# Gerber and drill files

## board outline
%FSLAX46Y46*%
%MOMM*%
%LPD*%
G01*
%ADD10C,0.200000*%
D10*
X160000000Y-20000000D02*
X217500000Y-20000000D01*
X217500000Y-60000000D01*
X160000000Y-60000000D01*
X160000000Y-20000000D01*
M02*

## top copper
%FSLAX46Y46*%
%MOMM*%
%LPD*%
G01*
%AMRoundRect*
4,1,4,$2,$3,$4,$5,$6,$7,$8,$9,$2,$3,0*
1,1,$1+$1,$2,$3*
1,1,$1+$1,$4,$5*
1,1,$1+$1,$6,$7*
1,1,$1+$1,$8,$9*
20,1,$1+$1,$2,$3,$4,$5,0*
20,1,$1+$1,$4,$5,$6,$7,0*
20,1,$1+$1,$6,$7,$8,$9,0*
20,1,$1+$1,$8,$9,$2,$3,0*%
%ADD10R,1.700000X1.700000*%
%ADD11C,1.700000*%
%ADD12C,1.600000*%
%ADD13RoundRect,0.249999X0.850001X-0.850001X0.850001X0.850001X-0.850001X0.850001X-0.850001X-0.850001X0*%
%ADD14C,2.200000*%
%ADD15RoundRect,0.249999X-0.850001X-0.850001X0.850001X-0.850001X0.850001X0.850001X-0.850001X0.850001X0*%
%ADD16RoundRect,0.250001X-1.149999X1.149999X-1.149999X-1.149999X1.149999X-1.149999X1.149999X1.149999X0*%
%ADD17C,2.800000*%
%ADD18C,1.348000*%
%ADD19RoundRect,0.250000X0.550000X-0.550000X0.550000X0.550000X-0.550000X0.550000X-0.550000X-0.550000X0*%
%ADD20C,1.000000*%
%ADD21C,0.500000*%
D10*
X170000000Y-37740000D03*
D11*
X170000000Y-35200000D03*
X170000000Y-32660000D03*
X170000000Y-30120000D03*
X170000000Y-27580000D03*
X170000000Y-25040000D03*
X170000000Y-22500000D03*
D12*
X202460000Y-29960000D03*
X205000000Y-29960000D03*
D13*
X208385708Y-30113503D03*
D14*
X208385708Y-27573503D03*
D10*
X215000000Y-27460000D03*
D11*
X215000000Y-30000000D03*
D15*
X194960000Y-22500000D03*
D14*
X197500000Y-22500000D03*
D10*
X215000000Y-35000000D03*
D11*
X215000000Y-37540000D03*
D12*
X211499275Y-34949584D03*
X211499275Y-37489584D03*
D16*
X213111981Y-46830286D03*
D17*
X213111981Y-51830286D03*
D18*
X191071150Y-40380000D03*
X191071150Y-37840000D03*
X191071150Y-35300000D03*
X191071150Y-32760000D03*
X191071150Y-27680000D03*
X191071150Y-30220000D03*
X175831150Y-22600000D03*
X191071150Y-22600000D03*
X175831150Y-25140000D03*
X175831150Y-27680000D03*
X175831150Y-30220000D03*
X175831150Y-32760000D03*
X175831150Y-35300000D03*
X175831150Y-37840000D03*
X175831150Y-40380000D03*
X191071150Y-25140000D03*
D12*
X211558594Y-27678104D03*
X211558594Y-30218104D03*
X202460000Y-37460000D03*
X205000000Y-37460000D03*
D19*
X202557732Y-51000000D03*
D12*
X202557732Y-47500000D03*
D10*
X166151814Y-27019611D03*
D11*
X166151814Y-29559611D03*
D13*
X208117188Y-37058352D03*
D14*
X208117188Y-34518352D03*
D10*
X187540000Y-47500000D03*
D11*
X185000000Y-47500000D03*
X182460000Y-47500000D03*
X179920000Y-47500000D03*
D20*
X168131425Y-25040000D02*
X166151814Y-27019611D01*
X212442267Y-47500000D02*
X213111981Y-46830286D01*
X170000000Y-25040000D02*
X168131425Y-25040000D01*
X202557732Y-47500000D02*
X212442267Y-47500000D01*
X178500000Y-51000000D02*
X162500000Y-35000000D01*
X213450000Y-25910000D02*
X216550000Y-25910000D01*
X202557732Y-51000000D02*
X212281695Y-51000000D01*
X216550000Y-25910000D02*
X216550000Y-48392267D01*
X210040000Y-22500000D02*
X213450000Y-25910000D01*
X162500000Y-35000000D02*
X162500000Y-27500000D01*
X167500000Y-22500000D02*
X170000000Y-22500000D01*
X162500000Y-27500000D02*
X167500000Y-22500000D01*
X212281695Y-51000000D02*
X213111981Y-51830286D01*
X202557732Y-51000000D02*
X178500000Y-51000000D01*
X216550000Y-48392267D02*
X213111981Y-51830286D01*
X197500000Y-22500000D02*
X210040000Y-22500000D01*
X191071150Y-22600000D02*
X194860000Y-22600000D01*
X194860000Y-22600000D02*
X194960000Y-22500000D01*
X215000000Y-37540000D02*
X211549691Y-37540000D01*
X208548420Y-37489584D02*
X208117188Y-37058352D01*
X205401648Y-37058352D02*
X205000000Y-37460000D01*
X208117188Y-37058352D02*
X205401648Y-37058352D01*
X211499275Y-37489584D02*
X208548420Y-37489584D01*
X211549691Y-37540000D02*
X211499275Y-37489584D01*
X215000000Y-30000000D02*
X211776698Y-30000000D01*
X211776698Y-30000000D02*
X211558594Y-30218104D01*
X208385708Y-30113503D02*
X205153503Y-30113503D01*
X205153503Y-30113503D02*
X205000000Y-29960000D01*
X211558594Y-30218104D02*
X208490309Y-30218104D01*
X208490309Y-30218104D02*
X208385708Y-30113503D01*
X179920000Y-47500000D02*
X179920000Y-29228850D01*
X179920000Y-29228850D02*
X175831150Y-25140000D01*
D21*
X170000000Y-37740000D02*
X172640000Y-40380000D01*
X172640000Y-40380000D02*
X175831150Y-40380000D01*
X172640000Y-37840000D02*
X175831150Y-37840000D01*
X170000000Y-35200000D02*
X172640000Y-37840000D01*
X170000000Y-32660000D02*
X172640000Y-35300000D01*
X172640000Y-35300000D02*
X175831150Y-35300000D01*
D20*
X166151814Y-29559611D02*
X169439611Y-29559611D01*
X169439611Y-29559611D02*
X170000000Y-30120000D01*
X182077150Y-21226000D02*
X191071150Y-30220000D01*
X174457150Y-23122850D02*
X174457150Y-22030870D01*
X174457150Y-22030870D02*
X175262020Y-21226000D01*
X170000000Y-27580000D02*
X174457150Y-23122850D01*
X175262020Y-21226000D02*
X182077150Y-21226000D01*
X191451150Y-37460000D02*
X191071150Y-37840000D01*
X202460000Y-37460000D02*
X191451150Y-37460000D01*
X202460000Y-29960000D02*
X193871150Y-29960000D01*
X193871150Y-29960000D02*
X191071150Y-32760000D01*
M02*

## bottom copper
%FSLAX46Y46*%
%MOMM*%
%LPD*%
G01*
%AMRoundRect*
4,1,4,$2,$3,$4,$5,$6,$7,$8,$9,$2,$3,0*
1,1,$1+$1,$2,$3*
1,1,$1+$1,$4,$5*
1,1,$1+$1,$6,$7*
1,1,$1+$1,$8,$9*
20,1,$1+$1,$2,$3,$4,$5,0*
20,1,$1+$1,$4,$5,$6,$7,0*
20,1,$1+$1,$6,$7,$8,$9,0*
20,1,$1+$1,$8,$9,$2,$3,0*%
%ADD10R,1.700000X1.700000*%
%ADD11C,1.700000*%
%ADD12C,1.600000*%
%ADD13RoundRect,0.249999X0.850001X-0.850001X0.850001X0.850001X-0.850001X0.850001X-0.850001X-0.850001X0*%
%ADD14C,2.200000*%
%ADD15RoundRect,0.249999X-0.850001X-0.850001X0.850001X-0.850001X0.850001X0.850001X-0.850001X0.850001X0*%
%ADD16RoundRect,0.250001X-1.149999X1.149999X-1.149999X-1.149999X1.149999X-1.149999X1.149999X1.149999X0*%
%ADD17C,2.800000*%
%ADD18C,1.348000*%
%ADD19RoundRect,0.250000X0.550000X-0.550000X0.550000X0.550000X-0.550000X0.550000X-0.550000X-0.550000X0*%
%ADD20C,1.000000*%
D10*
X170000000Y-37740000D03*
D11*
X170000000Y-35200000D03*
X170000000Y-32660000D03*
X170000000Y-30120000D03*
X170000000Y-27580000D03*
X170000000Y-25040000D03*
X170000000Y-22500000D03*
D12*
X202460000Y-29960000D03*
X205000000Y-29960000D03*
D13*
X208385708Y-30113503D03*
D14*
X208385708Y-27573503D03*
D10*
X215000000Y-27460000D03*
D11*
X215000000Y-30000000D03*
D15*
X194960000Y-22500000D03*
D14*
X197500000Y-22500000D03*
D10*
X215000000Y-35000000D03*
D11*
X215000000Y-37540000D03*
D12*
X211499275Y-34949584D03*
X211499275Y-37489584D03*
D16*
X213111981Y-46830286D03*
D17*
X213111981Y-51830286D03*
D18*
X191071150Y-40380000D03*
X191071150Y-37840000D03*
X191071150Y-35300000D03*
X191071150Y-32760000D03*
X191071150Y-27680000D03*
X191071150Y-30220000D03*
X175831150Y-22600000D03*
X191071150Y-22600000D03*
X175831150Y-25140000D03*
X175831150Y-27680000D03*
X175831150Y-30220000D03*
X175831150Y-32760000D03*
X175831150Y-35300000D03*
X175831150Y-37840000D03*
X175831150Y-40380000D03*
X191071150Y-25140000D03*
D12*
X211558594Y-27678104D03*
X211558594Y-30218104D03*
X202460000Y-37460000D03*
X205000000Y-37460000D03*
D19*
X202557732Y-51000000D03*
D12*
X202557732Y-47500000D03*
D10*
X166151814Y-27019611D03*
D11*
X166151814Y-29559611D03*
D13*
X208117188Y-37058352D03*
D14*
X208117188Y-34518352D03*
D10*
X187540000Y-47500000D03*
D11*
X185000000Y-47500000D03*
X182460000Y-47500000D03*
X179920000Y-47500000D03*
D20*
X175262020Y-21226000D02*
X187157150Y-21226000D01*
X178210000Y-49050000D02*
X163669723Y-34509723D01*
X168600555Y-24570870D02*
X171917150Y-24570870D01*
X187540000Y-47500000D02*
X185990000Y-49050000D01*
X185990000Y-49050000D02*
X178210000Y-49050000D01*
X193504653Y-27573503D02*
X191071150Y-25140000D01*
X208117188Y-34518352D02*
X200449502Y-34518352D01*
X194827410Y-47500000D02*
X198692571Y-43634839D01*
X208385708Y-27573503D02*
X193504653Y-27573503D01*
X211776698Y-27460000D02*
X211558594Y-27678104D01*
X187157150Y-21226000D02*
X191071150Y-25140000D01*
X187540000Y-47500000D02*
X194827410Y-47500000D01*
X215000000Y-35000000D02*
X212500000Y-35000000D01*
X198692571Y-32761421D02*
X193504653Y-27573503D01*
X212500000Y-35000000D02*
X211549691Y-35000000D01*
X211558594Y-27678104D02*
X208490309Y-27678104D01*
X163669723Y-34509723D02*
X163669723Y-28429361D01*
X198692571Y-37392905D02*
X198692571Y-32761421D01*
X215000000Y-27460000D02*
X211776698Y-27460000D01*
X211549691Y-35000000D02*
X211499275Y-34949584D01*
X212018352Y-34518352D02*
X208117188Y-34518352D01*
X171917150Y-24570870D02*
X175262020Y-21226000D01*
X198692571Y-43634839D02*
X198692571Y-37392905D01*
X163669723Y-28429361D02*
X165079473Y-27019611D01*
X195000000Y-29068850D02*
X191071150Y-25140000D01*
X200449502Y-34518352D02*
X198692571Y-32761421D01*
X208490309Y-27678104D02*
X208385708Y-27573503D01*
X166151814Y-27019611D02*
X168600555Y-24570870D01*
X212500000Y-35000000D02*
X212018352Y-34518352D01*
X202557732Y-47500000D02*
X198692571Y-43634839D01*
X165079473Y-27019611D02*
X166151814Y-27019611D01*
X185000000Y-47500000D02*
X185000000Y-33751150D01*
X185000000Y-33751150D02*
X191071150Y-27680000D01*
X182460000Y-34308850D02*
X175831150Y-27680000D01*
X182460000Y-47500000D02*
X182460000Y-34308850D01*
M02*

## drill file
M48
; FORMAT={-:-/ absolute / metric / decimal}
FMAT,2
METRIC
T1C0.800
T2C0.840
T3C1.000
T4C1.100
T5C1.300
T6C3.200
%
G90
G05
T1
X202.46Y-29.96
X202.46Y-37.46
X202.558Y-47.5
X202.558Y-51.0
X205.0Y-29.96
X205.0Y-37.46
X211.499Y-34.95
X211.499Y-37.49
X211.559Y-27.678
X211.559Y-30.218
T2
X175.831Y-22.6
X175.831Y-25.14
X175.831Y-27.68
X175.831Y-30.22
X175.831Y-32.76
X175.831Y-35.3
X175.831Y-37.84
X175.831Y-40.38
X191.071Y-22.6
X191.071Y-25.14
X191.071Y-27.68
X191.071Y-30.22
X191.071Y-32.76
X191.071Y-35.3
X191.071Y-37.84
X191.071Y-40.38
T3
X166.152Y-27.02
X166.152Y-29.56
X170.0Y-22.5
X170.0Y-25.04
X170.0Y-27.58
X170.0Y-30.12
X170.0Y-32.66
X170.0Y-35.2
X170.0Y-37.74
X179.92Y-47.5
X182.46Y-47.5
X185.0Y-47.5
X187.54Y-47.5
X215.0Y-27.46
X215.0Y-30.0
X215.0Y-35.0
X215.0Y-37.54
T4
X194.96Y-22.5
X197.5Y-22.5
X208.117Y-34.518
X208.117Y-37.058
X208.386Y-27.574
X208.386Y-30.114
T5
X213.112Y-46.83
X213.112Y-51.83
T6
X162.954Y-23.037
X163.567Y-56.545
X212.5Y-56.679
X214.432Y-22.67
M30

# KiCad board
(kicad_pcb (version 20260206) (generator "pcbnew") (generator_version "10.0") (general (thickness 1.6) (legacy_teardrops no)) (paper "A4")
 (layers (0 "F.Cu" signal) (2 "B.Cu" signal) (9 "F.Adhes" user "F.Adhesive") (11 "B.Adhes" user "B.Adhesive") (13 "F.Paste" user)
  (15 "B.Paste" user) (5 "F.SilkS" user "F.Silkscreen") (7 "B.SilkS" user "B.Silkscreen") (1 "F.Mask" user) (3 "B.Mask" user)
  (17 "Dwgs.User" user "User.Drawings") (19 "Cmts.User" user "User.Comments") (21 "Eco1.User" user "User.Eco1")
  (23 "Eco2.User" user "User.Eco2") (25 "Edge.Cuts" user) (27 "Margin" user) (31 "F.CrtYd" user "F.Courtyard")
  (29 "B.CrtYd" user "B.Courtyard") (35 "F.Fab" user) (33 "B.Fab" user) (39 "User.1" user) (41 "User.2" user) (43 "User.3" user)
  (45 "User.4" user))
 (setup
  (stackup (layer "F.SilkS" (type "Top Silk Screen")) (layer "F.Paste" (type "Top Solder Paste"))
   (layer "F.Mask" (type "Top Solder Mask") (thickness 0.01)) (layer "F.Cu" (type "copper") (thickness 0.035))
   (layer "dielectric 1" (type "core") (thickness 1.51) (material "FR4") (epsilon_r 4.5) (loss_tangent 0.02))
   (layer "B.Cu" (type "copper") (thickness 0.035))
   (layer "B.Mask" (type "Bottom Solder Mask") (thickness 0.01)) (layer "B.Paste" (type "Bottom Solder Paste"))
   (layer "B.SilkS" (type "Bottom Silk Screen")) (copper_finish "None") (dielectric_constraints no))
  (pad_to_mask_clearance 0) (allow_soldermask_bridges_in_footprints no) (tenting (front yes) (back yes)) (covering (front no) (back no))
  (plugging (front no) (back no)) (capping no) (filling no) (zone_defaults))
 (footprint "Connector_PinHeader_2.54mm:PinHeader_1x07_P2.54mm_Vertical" (layer "F.Cu") (at 170 37.74 180)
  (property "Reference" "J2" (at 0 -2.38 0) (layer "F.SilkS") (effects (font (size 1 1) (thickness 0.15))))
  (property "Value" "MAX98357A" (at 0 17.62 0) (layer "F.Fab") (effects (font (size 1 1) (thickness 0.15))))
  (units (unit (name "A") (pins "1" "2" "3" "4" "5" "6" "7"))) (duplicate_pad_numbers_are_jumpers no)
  (pad "1" thru_hole rect (at 0 0 180) (size 1.7 1.7) (drill 1) (layers "*.Cu" "*.Mask") (remove_unused_layers no) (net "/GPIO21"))
  (pad "2" thru_hole circle (at 0 2.54 180) (size 1.7 1.7) (drill 1) (layers "*.Cu" "*.Mask") (remove_unused_layers no) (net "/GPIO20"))
  (pad "3" thru_hole circle (at 0 5.08 180) (size 1.7 1.7) (drill 1) (layers "*.Cu" "*.Mask") (remove_unused_layers no) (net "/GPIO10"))
  (pad "4" thru_hole circle (at 0 7.62 180) (size 1.7 1.7) (drill 1) (layers "*.Cu" "*.Mask") (remove_unused_layers no)
   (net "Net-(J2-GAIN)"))
  (pad "5" thru_hole circle (at 0 10.16 180) (size 1.7 1.7) (drill 1) (layers "*.Cu" "*.Mask") (remove_unused_layers no) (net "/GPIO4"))
  (pad "6" thru_hole circle (at 0 12.7 180) (size 1.7 1.7) (drill 1) (layers "*.Cu" "*.Mask") (remove_unused_layers no) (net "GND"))
  (pad "7" thru_hole circle (at 0 15.24 180) (size 1.7 1.7) (drill 1) (layers "*.Cu" "*.Mask") (remove_unused_layers no) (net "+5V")))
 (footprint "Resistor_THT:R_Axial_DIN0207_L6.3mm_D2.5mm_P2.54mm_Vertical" (layer "F.Cu") (at 202.46 29.96)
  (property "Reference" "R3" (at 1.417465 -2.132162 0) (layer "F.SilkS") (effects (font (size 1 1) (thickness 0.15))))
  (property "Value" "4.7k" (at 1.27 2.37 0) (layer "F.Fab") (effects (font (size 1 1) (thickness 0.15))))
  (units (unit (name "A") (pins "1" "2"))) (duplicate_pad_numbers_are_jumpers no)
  (pad "1" thru_hole circle (at 0 0) (size 1.6 1.6) (drill 0.8) (layers "*.Cu" "*.Mask") (remove_unused_layers no) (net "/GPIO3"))
  (pad "2" thru_hole circle (at 2.54 0) (size 1.6 1.6) (drill 0.8) (layers "*.Cu" "*.Mask") (remove_unused_layers no) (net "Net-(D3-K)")))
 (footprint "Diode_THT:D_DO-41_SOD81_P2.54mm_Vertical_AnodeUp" (layer "F.Cu") (at 208.385708 30.113503 90)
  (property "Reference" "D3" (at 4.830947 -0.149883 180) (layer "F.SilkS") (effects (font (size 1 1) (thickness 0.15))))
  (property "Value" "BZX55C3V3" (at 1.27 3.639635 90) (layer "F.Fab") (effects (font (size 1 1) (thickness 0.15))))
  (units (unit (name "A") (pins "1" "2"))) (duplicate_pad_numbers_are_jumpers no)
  (pad "1" thru_hole roundrect (at 0 0 90) (size 2.2 2.2) (drill 1.1) (layers "*.Cu" "*.Mask") (remove_unused_layers no)
   (roundrect_rratio 0.113636) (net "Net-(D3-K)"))
  (pad "2" thru_hole circle (at 2.54 0 90) (size 2.2 2.2) (drill 1.1) (layers "*.Cu" "*.Mask") (remove_unused_layers no) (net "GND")))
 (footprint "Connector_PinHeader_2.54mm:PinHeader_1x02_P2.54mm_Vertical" (layer "F.Cu") (at 215 27.46)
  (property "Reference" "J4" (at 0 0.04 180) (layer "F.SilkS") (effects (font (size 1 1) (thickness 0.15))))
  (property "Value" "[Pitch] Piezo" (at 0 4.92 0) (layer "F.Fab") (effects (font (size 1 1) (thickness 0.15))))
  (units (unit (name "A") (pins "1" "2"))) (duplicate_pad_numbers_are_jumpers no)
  (pad "1" thru_hole rect (at 0 0) (size 1.7 1.7) (drill 1) (layers "*.Cu" "*.Mask") (remove_unused_layers no) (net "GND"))
  (pad "2" thru_hole circle (at 0 2.54) (size 1.7 1.7) (drill 1) (layers "*.Cu" "*.Mask") (remove_unused_layers no) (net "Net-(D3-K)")))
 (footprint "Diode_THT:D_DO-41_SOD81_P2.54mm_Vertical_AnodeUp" (layer "F.Cu") (at 194.96 22.5)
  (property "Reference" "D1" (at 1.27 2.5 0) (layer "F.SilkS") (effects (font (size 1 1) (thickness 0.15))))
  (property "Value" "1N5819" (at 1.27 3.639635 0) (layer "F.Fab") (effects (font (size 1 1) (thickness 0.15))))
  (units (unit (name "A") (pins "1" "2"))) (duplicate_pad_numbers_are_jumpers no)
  (pad "1" thru_hole roundrect (at 0 0) (size 2.2 2.2) (drill 1.1) (layers "*.Cu" "*.Mask") (remove_unused_layers no)
   (roundrect_rratio 0.113636) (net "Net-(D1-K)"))
  (pad "2" thru_hole circle (at 2.54 0) (size 2.2 2.2) (drill 1.1) (layers "*.Cu" "*.Mask") (remove_unused_layers no) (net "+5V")))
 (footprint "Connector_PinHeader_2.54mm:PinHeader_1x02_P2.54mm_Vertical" (layer "F.Cu") (at 215 35)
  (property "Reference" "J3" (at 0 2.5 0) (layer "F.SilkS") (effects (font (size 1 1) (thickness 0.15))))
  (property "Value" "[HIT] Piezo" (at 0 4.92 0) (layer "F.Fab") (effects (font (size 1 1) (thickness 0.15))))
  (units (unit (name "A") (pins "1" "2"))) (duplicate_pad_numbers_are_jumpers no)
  (pad "1" thru_hole rect (at 0 0) (size 1.7 1.7) (drill 1) (layers "*.Cu" "*.Mask") (remove_unused_layers no) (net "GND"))
  (pad "2" thru_hole circle (at 0 2.54) (size 1.7 1.7) (drill 1) (layers "*.Cu" "*.Mask") (remove_unused_layers no) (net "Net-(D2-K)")))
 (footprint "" (layer "F.Cu") (at 163.567285 56.544557)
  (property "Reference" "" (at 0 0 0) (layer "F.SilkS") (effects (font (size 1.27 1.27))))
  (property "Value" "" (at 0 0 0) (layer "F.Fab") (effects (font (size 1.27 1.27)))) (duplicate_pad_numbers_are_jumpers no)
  (pad "" np_thru_hole circle (at 0 0) (size 3.2 3.2) (drill 3.2) (layers "*.Cu" "*.Mask")))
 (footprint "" (layer "F.Cu") (at 212.5 56.678691)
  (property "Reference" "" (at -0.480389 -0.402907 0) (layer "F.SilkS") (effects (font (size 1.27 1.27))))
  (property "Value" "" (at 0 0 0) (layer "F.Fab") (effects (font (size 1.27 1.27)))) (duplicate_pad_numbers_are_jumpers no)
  (pad "" np_thru_hole circle (at 0 0) (size 3.2 3.2) (drill 3.2) (layers "*.Cu" "*.Mask")))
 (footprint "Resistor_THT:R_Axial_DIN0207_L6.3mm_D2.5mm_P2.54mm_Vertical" (layer "F.Cu") (at 211.499275 34.949584 -90)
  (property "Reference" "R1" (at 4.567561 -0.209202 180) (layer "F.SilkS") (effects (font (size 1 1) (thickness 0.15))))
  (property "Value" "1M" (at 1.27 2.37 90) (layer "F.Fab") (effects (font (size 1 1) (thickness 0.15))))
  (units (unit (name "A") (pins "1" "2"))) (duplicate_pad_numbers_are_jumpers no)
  (pad "1" thru_hole circle (at 0 0 270) (size 1.6 1.6) (drill 0.8) (layers "*.Cu" "*.Mask") (remove_unused_layers no) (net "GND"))
  (pad "2" thru_hole circle (at 2.54 0 270) (size 1.6 1.6) (drill 0.8) (layers "*.Cu" "*.Mask") (remove_unused_layers no) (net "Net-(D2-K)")))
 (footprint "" (layer "F.Cu") (at 162.954392 23.037208)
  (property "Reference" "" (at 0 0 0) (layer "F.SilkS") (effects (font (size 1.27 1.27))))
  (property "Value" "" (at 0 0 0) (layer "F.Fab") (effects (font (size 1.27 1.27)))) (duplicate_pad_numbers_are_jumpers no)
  (pad "" np_thru_hole circle (at 0 0) (size 3.2 3.2) (drill 3.2) (layers "*.Cu" "*.Mask")))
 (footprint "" (layer "F.Cu") (at 214.431967 22.67046)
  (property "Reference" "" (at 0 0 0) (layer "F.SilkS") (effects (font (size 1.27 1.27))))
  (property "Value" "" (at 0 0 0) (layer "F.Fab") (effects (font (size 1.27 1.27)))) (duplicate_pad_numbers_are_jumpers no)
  (pad "" np_thru_hole circle (at 0 0) (size 3.2 3.2) (drill 3.2) (layers "*.Cu" "*.Mask")))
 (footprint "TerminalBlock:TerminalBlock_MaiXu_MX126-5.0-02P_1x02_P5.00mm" (layer "F.Cu") (at 213.111981 46.830286 -90)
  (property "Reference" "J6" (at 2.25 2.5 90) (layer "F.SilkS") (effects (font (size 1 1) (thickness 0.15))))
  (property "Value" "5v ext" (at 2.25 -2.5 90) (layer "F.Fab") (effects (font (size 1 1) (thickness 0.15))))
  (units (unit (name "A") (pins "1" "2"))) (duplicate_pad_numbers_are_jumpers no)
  (pad "1" thru_hole roundrect (at 0 0 270) (size 2.8 2.8) (drill 1.3) (layers "*.Cu" "*.Mask") (remove_unused_layers no)
   (roundrect_rratio 0.089286) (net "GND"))
  (pad "2" thru_hole circle (at 5 0 270) (size 2.8 2.8) (drill 1.3) (layers "*.Cu" "*.Mask") (remove_unused_layers no) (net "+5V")))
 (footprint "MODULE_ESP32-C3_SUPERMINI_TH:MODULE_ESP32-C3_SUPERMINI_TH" (layer "F.Cu") (at 183.45115 32.5)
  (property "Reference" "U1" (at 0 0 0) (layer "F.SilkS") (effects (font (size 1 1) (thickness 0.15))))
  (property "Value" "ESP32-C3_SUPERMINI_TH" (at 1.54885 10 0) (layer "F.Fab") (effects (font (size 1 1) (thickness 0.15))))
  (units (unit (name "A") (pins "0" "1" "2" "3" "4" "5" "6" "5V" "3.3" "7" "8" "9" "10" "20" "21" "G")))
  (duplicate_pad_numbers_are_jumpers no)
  (pad "0" thru_hole circle (at 7.62 7.88) (size 1.348 1.348) (drill 0.84) (layers "*.Cu" "*.Mask") (remove_unused_layers no)
   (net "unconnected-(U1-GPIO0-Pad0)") (solder_mask_margin 0.102))
  (pad "1" thru_hole circle (at 7.62 5.34) (size 1.348 1.348) (drill 0.84) (layers "*.Cu" "*.Mask") (remove_unused_layers no) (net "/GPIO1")
   (solder_mask_margin 0.102))
  (pad "2" thru_hole circle (at 7.62 2.8) (size 1.348 1.348) (drill 0.84) (layers "*.Cu" "*.Mask") (remove_unused_layers no)
   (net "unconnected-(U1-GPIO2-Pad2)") (solder_mask_margin 0.102))
  (pad "3" thru_hole circle (at 7.62 0.26) (size 1.348 1.348) (drill 0.84) (layers "*.Cu" "*.Mask") (remove_unused_layers no) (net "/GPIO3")
   (solder_mask_margin 0.102))
  (pad "3.3" thru_hole circle (at 7.62 -4.82) (size 1.348 1.348) (drill 0.84) (layers "*.Cu" "*.Mask") (remove_unused_layers no)
   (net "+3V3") (solder_mask_margin 0.102))
  (pad "4" thru_hole circle (at 7.62 -2.28) (size 1.348 1.348) (drill 0.84) (layers "*.Cu" "*.Mask") (remove_unused_layers no)
   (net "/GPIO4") (solder_mask_margin 0.102))
  (pad "5" thru_hole circle (at -7.62 -9.9) (size 1.348 1.348) (drill 0.84) (layers "*.Cu" "*.Mask") (remove_unused_layers no)
   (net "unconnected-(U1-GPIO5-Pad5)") (solder_mask_margin 0.102))
  (pad "5V" thru_hole circle (at 7.62 -9.9) (size 1.348 1.348) (drill 0.84) (layers "*.Cu" "*.Mask") (remove_unused_layers no)
   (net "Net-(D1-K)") (solder_mask_margin 0.102))
  (pad "6" thru_hole circle (at -7.62 -7.36) (size 1.348 1.348) (drill 0.84) (layers "*.Cu" "*.Mask") (remove_unused_layers no) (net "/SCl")
   (solder_mask_margin 0.102))
  (pad "7" thru_hole circle (at -7.62 -4.82) (size 1.348 1.348) (drill 0.84) (layers "*.Cu" "*.Mask") (remove_unused_layers no) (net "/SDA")
   (solder_mask_margin 0.102))
  (pad "8" thru_hole circle (at -7.62 -2.28) (size 1.348 1.348) (drill 0.84) (layers "*.Cu" "*.Mask") (remove_unused_layers no)
   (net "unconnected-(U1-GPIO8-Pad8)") (solder_mask_margin 0.102))
  (pad "9" thru_hole circle (at -7.62 0.26) (size 1.348 1.348) (drill 0.84) (layers "*.Cu" "*.Mask") (remove_unused_layers no)
   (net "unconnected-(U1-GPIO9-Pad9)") (solder_mask_margin 0.102))
  (pad "10" thru_hole circle (at -7.62 2.8) (size 1.348 1.348) (drill 0.84) (layers "*.Cu" "*.Mask") (remove_unused_layers no)
   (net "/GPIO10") (solder_mask_margin 0.102))
  (pad "20" thru_hole circle (at -7.62 5.34) (size 1.348 1.348) (drill 0.84) (layers "*.Cu" "*.Mask") (remove_unused_layers no)
   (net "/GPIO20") (solder_mask_margin 0.102))
  (pad "21" thru_hole circle (at -7.62 7.88) (size 1.348 1.348) (drill 0.84) (layers "*.Cu" "*.Mask") (remove_unused_layers no)
   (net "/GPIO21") (solder_mask_margin 0.102))
  (pad "G" thru_hole circle (at 7.62 -7.36) (size 1.348 1.348) (drill 0.84) (layers "*.Cu" "*.Mask") (remove_unused_layers no) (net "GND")
   (solder_mask_margin 0.102)))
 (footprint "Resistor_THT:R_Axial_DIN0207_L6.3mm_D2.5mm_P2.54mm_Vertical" (layer "F.Cu") (at 211.558594 27.678104 -90)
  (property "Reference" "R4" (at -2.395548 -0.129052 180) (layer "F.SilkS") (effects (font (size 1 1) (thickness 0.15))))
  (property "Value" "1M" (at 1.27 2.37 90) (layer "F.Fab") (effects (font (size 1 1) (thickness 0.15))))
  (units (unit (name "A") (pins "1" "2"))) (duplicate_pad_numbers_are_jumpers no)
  (pad "1" thru_hole circle (at 0 0 270) (size 1.6 1.6) (drill 0.8) (layers "*.Cu" "*.Mask") (remove_unused_layers no) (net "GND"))
  (pad "2" thru_hole circle (at 2.54 0 270) (size 1.6 1.6) (drill 0.8) (layers "*.Cu" "*.Mask") (remove_unused_layers no) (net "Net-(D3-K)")))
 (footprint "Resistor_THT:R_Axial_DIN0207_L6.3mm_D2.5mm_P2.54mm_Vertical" (layer "F.Cu") (at 202.46 37.46)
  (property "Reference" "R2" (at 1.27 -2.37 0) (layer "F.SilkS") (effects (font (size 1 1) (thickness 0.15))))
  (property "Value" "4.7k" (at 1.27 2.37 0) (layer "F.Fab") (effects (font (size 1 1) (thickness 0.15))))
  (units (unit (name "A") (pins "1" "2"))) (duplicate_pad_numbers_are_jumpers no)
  (pad "1" thru_hole circle (at 0 0) (size 1.6 1.6) (drill 0.8) (layers "*.Cu" "*.Mask") (remove_unused_layers no) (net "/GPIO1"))
  (pad "2" thru_hole circle (at 2.54 0) (size 1.6 1.6) (drill 0.8) (layers "*.Cu" "*.Mask") (remove_unused_layers no) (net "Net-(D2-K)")))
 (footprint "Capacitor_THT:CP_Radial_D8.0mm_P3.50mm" (layer "F.Cu") (at 202.557732 51 90)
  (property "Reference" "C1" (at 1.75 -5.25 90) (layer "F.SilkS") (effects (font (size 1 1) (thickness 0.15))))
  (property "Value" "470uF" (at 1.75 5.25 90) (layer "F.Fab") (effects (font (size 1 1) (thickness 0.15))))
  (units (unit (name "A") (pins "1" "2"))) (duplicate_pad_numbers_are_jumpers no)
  (pad "1" thru_hole roundrect (at 0 0 90) (size 1.6 1.6) (drill 0.8) (layers "*.Cu" "*.Mask") (remove_unused_layers no)
   (roundrect_rratio 0.15625) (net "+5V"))
  (pad "2" thru_hole circle (at 3.5 0 90) (size 1.6 1.6) (drill 0.8) (layers "*.Cu" "*.Mask") (remove_unused_layers no) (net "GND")))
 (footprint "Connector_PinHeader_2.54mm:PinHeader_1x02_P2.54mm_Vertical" (layer "F.Cu") (at 166.151814 27.019611)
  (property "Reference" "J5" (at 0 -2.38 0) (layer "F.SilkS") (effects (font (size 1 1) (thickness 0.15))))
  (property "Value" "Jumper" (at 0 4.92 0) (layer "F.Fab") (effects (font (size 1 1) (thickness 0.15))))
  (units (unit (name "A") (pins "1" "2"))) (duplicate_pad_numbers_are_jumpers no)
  (pad "1" thru_hole rect (at 0 0) (size 1.7 1.7) (drill 1) (layers "*.Cu" "*.Mask") (remove_unused_layers no) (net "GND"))
  (pad "2" thru_hole circle (at 0 2.54) (size 1.7 1.7) (drill 1) (layers "*.Cu" "*.Mask") (remove_unused_layers no) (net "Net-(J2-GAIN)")))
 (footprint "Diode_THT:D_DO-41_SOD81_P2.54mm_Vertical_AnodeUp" (layer "F.Cu") (at 208.117188 37.058352 90)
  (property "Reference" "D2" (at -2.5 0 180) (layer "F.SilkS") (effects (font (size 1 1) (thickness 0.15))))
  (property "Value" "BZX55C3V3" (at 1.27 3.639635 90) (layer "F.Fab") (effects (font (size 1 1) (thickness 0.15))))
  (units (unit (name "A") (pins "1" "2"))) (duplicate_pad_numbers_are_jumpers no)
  (pad "1" thru_hole roundrect (at 0 0 90) (size 2.2 2.2) (drill 1.1) (layers "*.Cu" "*.Mask") (remove_unused_layers no)
   (roundrect_rratio 0.113636) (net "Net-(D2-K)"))
  (pad "2" thru_hole circle (at 2.54 0 90) (size 2.2 2.2) (drill 1.1) (layers "*.Cu" "*.Mask") (remove_unused_layers no) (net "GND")))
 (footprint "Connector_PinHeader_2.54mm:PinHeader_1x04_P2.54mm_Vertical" (layer "B.Cu") (at 187.54 47.5 90)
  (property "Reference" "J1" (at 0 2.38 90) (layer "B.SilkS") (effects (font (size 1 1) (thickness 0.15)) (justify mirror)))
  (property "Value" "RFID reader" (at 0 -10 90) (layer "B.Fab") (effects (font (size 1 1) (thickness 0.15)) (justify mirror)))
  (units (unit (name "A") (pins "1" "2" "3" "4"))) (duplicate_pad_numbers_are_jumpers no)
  (pad "1" thru_hole rect (at 0 0 90) (size 1.7 1.7) (drill 1) (layers "*.Cu" "*.Mask") (remove_unused_layers no) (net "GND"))
  (pad "2" thru_hole circle (at 0 -2.54 90) (size 1.7 1.7) (drill 1) (layers "*.Cu" "*.Mask") (remove_unused_layers no) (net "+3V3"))
  (pad "3" thru_hole circle (at 0 -5.08 90) (size 1.7 1.7) (drill 1) (layers "*.Cu" "*.Mask") (remove_unused_layers no) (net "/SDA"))
  (pad "4" thru_hole circle (at 0 -7.62 90) (size 1.7 1.7) (drill 1) (layers "*.Cu" "*.Mask") (remove_unused_layers no) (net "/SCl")))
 (gr_rect (start 160 20) (end 217.5 60) (stroke (width 0.2) (type solid)) (fill no) (layer "Edge.Cuts"))
 (segment (start 168.131425 25.04) (end 166.151814 27.019611) (width 1) (layer "F.Cu") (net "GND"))
 (segment (start 212.442267 47.5) (end 213.111981 46.830286) (width 1) (layer "F.Cu") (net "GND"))
 (segment (start 170 25.04) (end 168.131425 25.04) (width 1) (layer "F.Cu") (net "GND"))
 (segment (start 202.557732 47.5) (end 212.442267 47.5) (width 1) (layer "F.Cu") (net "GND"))
 (segment (start 175.26202 21.226) (end 187.15715 21.226) (width 1) (layer "B.Cu") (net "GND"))
 (segment (start 178.21 49.05) (end 163.669723 34.509723) (width 1) (layer "B.Cu") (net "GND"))
 (segment (start 168.600555 24.57087) (end 171.91715 24.57087) (width 1) (layer "B.Cu") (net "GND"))
 (segment (start 187.54 47.5) (end 185.99 49.05) (width 1) (layer "B.Cu") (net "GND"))
 (segment (start 185.99 49.05) (end 178.21 49.05) (width 1) (layer "B.Cu") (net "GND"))
 (segment (start 193.504653 27.573503) (end 191.07115 25.14) (width 1) (layer "B.Cu") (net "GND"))
 (segment (start 208.117188 34.518352) (end 200.449502 34.518352) (width 1) (layer "B.Cu") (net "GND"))
 (segment (start 194.82741 47.5) (end 198.692571 43.634839) (width 1) (layer "B.Cu") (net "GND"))
 (segment (start 208.385708 27.573503) (end 193.504653 27.573503) (width 1) (layer "B.Cu") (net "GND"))
 (segment (start 211.776698 27.46) (end 211.558594 27.678104) (width 1) (layer "B.Cu") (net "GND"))
 (segment (start 187.15715 21.226) (end 191.07115 25.14) (width 1) (layer "B.Cu") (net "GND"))
 (segment (start 187.54 47.5) (end 194.82741 47.5) (width 1) (layer "B.Cu") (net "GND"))
 (segment (start 215 35) (end 212.5 35) (width 1) (layer "B.Cu") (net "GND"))
 (segment (start 198.692571 32.761421) (end 193.504653 27.573503) (width 1) (layer "B.Cu") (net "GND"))
 (segment (start 212.5 35) (end 211.549691 35) (width 1) (layer "B.Cu") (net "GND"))
 (segment (start 211.558594 27.678104) (end 208.490309 27.678104) (width 1) (layer "B.Cu") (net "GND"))
 (segment (start 163.669723 34.509723) (end 163.669723 28.429361) (width 1) (layer "B.Cu") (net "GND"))
 (segment (start 198.692571 37.392905) (end 198.692571 32.761421) (width 1) (layer "B.Cu") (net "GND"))
 (segment (start 215 27.46) (end 211.776698 27.46) (width 1) (layer "B.Cu") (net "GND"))
 (segment (start 211.549691 35) (end 211.499275 34.949584) (width 1) (layer "B.Cu") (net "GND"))
 (segment (start 212.018352 34.518352) (end 208.117188 34.518352) (width 1) (layer "B.Cu") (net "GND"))
 (segment (start 171.91715 24.57087) (end 175.26202 21.226) (width 1) (layer "B.Cu") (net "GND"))
 (segment (start 198.692571 43.634839) (end 198.692571 37.392905) (width 1) (layer "B.Cu") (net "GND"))
 (segment (start 163.669723 28.429361) (end 165.079473 27.019611) (width 1) (layer "B.Cu") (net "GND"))
 (segment (start 195 29.06885) (end 191.07115 25.14) (width 1) (layer "B.Cu") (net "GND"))
 (segment (start 200.449502 34.518352) (end 198.692571 32.761421) (width 1) (layer "B.Cu") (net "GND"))
 (segment (start 208.490309 27.678104) (end 208.385708 27.573503) (width 1) (layer "B.Cu") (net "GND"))
 (segment (start 166.151814 27.019611) (end 168.600555 24.57087) (width 1) (layer "B.Cu") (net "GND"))
 (segment (start 212.5 35) (end 212.018352 34.518352) (width 1) (layer "B.Cu") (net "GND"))
 (segment (start 202.557732 47.5) (end 198.692571 43.634839) (width 1) (layer "B.Cu") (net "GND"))
 (segment (start 165.079473 27.019611) (end 166.151814 27.019611) (width 1) (layer "B.Cu") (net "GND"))
 (segment (start 178.5 51) (end 162.5 35) (width 1) (layer "F.Cu") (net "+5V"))
 (segment (start 213.45 25.91) (end 216.55 25.91) (width 1) (layer "F.Cu") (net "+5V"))
 (segment (start 202.557732 51) (end 212.281695 51) (width 1) (layer "F.Cu") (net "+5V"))
 (segment (start 216.55 25.91) (end 216.55 48.392267) (width 1) (layer "F.Cu") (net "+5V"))
 (segment (start 210.04 22.5) (end 213.45 25.91) (width 1) (layer "F.Cu") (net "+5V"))
 (segment (start 162.5 35) (end 162.5 27.5) (width 1) (layer "F.Cu") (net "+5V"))
 (segment (start 167.5 22.5) (end 170 22.5) (width 1) (layer "F.Cu") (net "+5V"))
 (segment (start 162.5 27.5) (end 167.5 22.5) (width 1) (layer "F.Cu") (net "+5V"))
 (segment (start 212.281695 51) (end 213.111981 51.830286) (width 1) (layer "F.Cu") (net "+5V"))
 (segment (start 202.557732 51) (end 178.5 51) (width 1) (layer "F.Cu") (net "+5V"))
 (segment (start 216.55 48.392267) (end 213.111981 51.830286) (width 1) (layer "F.Cu") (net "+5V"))
 (segment (start 197.5 22.5) (end 210.04 22.5) (width 1) (layer "F.Cu") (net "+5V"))
 (segment (start 191.07115 22.6) (end 194.86 22.6) (width 1) (layer "F.Cu") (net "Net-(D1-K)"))
 (segment (start 194.86 22.6) (end 194.96 22.5) (width 1) (layer "F.Cu") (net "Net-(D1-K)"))
 (segment (start 215 37.54) (end 211.549691 37.54) (width 1) (layer "F.Cu") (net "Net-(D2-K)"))
 (segment (start 208.54842 37.489584) (end 208.117188 37.058352) (width 1) (layer "F.Cu") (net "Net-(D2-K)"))
 (segment (start 205.401648 37.058352) (end 205 37.46) (width 1) (layer "F.Cu") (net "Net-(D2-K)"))
 (segment (start 208.117188 37.058352) (end 205.401648 37.058352) (width 1) (layer "F.Cu") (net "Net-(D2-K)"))
 (segment (start 211.499275 37.489584) (end 208.54842 37.489584) (width 1) (layer "F.Cu") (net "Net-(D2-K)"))
 (segment (start 211.549691 37.54) (end 211.499275 37.489584) (width 1) (layer "F.Cu") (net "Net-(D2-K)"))
 (segment (start 215 30) (end 211.776698 30) (width 1) (layer "F.Cu") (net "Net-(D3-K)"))
 (segment (start 211.776698 30) (end 211.558594 30.218104) (width 1) (layer "F.Cu") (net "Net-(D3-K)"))
 (segment (start 208.385708 30.113503) (end 205.153503 30.113503) (width 1) (layer "F.Cu") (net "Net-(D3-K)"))
 (segment (start 205.153503 30.113503) (end 205 29.96) (width 1) (layer "F.Cu") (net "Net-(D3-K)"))
 (segment (start 211.558594 30.218104) (end 208.490309 30.218104) (width 1) (layer "F.Cu") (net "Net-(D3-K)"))
 (segment (start 208.490309 30.218104) (end 208.385708 30.113503) (width 1) (layer "F.Cu") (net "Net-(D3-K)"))
 (segment (start 179.92 47.5) (end 179.92 29.22885) (width 1) (layer "F.Cu") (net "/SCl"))
 (segment (start 179.92 29.22885) (end 175.83115 25.14) (width 1) (layer "F.Cu") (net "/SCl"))
 (segment (start 185 47.5) (end 185 33.75115) (width 1) (layer "B.Cu") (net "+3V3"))
 (segment (start 185 33.75115) (end 191.07115 27.68) (width 1) (layer "B.Cu") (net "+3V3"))
 (segment (start 182.46 34.30885) (end 175.83115 27.68) (width 1) (layer "B.Cu") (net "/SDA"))
 (segment (start 182.46 47.5) (end 182.46 34.30885) (width 1) (layer "B.Cu") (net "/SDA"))
 (segment (start 170 37.74) (end 172.64 40.38) (width 0.5) (layer "F.Cu") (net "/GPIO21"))
 (segment (start 172.64 40.38) (end 175.83115 40.38) (width 0.5) (layer "F.Cu") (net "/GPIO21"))
 (segment (start 172.64 37.84) (end 175.83115 37.84) (width 0.5) (layer "F.Cu") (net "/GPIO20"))
 (segment (start 170 35.2) (end 172.64 37.84) (width 0.5) (layer "F.Cu") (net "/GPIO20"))
 (segment (start 170 32.66) (end 172.64 35.3) (width 0.5) (layer "F.Cu") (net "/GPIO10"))
 (segment (start 172.64 35.3) (end 175.83115 35.3) (width 0.5) (layer "F.Cu") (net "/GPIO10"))
 (segment (start 166.151814 29.559611) (end 169.439611 29.559611) (width 1) (layer "F.Cu") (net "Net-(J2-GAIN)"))
 (segment (start 169.439611 29.559611) (end 170 30.12) (width 1) (layer "F.Cu") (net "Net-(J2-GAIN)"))
 (segment (start 182.07715 21.226) (end 191.07115 30.22) (width 1) (layer "F.Cu") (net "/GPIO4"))
 (segment (start 174.45715 23.12285) (end 174.45715 22.03087) (width 1) (layer "F.Cu") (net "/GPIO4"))
 (segment (start 174.45715 22.03087) (end 175.26202 21.226) (width 1) (layer "F.Cu") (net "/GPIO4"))
 (segment (start 170 27.58) (end 174.45715 23.12285) (width 1) (layer "F.Cu") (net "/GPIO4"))
 (segment (start 175.26202 21.226) (end 182.07715 21.226) (width 1) (layer "F.Cu") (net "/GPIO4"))
 (segment (start 191.45115 37.46) (end 191.07115 37.84) (width 1) (layer "F.Cu") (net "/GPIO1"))
 (segment (start 202.46 37.46) (end 191.45115 37.46) (width 1) (layer "F.Cu") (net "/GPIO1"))
 (segment (start 202.46 29.96) (end 193.87115 29.96) (width 1) (layer "F.Cu") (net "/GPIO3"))
 (segment (start 193.87115 29.96) (end 191.07115 32.76) (width 1) (layer "F.Cu") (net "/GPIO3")))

